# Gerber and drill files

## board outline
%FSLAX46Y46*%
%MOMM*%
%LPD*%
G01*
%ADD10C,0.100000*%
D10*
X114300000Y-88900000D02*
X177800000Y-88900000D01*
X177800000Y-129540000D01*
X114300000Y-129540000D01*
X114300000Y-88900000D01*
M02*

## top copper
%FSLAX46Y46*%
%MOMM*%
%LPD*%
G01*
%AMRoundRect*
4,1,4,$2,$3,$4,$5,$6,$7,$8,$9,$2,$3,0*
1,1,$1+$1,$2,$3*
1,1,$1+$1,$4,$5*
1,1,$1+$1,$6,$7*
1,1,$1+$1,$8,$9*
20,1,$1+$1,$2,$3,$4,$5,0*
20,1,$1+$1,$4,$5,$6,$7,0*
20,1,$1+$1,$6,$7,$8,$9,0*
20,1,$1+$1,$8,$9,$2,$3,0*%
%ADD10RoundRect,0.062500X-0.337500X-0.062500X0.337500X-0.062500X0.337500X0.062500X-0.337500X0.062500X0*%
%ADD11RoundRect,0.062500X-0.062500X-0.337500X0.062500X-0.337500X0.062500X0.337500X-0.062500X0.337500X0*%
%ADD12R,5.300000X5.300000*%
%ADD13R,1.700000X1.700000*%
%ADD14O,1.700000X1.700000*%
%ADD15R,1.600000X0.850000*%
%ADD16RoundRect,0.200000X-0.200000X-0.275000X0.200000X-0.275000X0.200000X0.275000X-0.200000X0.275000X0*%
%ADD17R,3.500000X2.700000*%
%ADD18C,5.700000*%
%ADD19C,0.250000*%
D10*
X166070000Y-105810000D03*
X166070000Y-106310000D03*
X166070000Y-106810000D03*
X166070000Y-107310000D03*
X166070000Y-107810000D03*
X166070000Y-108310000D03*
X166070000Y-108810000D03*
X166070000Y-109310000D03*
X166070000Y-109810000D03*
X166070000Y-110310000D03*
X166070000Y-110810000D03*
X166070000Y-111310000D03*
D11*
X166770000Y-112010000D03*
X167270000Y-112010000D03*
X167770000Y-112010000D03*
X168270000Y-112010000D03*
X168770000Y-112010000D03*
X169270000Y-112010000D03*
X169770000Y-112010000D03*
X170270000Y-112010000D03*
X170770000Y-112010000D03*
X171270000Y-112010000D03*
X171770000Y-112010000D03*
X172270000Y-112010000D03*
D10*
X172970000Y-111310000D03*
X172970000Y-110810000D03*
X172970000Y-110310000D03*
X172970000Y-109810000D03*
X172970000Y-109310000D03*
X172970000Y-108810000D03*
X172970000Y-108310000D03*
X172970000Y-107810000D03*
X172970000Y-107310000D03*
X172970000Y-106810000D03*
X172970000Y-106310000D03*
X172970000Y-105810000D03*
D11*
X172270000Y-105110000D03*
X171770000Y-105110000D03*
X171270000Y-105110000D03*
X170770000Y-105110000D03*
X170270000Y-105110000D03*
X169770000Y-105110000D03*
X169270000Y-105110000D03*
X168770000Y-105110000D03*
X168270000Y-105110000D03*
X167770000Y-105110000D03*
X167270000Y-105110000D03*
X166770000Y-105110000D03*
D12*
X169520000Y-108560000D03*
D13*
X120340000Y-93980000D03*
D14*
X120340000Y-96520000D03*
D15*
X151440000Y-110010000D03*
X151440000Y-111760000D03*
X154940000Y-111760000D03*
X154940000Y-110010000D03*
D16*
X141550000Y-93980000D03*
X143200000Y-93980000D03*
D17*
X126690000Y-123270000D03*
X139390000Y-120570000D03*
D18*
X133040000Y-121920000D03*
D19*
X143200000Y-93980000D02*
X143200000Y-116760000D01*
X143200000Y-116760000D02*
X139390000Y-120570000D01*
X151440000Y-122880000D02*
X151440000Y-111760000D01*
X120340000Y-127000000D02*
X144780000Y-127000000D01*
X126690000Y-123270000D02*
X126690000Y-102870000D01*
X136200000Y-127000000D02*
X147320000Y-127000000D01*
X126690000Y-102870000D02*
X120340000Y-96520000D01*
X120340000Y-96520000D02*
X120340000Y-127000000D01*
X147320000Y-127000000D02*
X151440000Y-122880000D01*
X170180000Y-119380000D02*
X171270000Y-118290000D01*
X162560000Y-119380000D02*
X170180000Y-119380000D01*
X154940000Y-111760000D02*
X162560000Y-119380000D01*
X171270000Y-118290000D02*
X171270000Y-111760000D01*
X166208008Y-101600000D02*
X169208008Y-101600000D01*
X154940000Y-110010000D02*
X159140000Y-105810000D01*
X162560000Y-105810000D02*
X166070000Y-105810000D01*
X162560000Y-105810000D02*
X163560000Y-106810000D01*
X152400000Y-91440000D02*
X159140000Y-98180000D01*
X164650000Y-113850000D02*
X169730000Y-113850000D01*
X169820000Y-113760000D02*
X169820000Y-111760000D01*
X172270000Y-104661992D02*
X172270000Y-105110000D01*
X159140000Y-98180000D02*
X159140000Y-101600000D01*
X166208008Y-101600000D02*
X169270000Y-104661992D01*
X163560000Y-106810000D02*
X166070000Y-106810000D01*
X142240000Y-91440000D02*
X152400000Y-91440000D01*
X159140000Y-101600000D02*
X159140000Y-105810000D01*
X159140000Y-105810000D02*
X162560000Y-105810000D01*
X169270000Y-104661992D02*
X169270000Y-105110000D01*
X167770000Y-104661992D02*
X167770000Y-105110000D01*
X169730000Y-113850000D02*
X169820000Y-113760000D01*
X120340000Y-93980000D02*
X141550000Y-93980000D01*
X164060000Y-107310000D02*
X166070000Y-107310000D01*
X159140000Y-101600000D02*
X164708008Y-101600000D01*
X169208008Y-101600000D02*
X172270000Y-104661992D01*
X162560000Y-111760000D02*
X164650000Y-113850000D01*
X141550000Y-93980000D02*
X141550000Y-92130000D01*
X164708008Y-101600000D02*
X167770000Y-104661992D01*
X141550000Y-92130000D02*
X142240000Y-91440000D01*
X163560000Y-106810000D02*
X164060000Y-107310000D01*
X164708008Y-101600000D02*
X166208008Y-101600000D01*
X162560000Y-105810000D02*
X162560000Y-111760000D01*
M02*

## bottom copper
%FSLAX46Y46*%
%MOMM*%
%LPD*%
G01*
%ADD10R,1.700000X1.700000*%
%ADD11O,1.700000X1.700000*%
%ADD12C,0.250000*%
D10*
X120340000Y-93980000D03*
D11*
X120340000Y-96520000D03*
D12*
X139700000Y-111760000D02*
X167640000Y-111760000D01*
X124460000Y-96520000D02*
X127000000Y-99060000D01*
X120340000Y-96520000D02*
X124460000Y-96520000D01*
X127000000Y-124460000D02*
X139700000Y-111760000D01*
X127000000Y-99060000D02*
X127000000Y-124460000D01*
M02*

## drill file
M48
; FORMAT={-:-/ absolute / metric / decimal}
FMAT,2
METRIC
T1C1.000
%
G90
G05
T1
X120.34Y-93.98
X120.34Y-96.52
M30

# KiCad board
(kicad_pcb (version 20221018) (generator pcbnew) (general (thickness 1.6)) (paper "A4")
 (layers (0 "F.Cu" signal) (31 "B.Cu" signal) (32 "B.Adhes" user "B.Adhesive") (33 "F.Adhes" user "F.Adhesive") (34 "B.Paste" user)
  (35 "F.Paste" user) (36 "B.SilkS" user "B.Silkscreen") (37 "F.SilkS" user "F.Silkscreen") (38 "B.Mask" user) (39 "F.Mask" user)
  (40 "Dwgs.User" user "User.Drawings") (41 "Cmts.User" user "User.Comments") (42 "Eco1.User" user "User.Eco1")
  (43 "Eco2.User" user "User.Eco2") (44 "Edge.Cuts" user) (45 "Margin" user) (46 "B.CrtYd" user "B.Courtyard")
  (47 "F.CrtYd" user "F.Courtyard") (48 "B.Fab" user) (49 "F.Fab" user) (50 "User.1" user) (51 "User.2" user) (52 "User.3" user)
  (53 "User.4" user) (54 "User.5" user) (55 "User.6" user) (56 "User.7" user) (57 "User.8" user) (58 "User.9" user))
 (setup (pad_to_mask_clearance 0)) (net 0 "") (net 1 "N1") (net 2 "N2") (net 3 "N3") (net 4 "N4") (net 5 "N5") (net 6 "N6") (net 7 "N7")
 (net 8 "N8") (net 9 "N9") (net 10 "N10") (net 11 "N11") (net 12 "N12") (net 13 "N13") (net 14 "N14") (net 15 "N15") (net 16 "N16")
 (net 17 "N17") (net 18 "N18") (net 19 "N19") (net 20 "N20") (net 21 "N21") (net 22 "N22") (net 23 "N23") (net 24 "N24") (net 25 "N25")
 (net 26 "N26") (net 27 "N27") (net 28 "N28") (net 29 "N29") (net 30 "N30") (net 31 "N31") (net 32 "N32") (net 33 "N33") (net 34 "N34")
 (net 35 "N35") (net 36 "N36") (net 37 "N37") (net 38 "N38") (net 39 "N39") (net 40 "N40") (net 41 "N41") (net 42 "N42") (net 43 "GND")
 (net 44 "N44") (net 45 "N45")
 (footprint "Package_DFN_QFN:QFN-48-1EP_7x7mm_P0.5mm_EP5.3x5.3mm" (layer "F.Cu") (at 169.52 108.56)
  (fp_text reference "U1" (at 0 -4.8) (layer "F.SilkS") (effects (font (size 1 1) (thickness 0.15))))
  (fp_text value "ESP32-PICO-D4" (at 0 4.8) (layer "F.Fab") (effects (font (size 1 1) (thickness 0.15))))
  (pad "" smd roundrect (at -1.98 -1.98) (size 1.07 1.07) (layers "F.Paste") (roundrect_rratio 0.233645))
  (pad "" smd roundrect (at -1.98 -0.66) (size 1.07 1.07) (layers "F.Paste") (roundrect_rratio 0.233645))
  (pad "" smd roundrect (at -1.98 0.66) (size 1.07 1.07) (layers "F.Paste") (roundrect_rratio 0.233645))
  (pad "" smd roundrect (at -1.98 1.98) (size 1.07 1.07) (layers "F.Paste") (roundrect_rratio 0.233645))
  (pad "" smd roundrect (at -0.66 -1.98) (size 1.07 1.07) (layers "F.Paste") (roundrect_rratio 0.233645))
  (pad "" smd roundrect (at -0.66 -0.66) (size 1.07 1.07) (layers "F.Paste") (roundrect_rratio 0.233645))
  (pad "" smd roundrect (at -0.66 0.66) (size 1.07 1.07) (layers "F.Paste") (roundrect_rratio 0.233645))
  (pad "" smd roundrect (at -0.66 1.98) (size 1.07 1.07) (layers "F.Paste") (roundrect_rratio 0.233645))
  (pad "" smd roundrect (at 0.66 -1.98) (size 1.07 1.07) (layers "F.Paste") (roundrect_rratio 0.233645))
  (pad "" smd roundrect (at 0.66 -0.66) (size 1.07 1.07) (layers "F.Paste") (roundrect_rratio 0.233645))
  (pad "" smd roundrect (at 0.66 0.66) (size 1.07 1.07) (layers "F.Paste") (roundrect_rratio 0.233645))
  (pad "" smd roundrect (at 0.66 1.98) (size 1.07 1.07) (layers "F.Paste") (roundrect_rratio 0.233645))
  (pad "" smd roundrect (at 1.98 -1.98) (size 1.07 1.07) (layers "F.Paste") (roundrect_rratio 0.233645))
  (pad "" smd roundrect (at 1.98 -0.66) (size 1.07 1.07) (layers "F.Paste") (roundrect_rratio 0.233645))
  (pad "" smd roundrect (at 1.98 0.66) (size 1.07 1.07) (layers "F.Paste") (roundrect_rratio 0.233645))
  (pad "" smd roundrect (at 1.98 1.98) (size 1.07 1.07) (layers "F.Paste") (roundrect_rratio 0.233645))
  (pad "1" smd roundrect (at -3.45 -2.75) (size 0.8 0.25) (layers "F.Cu" "F.Paste" "F.Mask") (roundrect_rratio 0.25) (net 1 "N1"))
  (pad "2" smd roundrect (at -3.45 -2.25) (size 0.8 0.25) (layers "F.Cu" "F.Paste" "F.Mask") (roundrect_rratio 0.25) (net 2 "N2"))
  (pad "3" smd roundrect (at -3.45 -1.75) (size 0.8 0.25) (layers "F.Cu" "F.Paste" "F.Mask") (roundrect_rratio 0.25) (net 1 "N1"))
  (pad "4" smd roundrect (at -3.45 -1.25) (size 0.8 0.25) (layers "F.Cu" "F.Paste" "F.Mask") (roundrect_rratio 0.25) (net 1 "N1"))
  (pad "5" smd roundrect (at -3.45 -0.75) (size 0.8 0.25) (layers "F.Cu" "F.Paste" "F.Mask") (roundrect_rratio 0.25) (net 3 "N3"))
  (pad "6" smd roundrect (at -3.45 -0.25) (size 0.8 0.25) (layers "F.Cu" "F.Paste" "F.Mask") (roundrect_rratio 0.25) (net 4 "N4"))
  (pad "7" smd roundrect (at -3.45 0.25) (size 0.8 0.25) (layers "F.Cu" "F.Paste" "F.Mask") (roundrect_rratio 0.25) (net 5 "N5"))
  (pad "8" smd roundrect (at -3.45 0.75) (size 0.8 0.25) (layers "F.Cu" "F.Paste" "F.Mask") (roundrect_rratio 0.25) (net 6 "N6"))
  (pad "9" smd roundrect (at -3.45 1.25) (size 0.8 0.25) (layers "F.Cu" "F.Paste" "F.Mask") (roundrect_rratio 0.25) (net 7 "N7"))
  (pad "10" smd roundrect (at -3.45 1.75) (size 0.8 0.25) (layers "F.Cu" "F.Paste" "F.Mask") (roundrect_rratio 0.25) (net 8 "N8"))
  (pad "11" smd roundrect (at -3.45 2.25) (size 0.8 0.25) (layers "F.Cu" "F.Paste" "F.Mask") (roundrect_rratio 0.25) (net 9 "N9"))
  (pad "12" smd roundrect (at -3.45 2.75) (size 0.8 0.25) (layers "F.Cu" "F.Paste" "F.Mask") (roundrect_rratio 0.25) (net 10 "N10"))
  (pad "13" smd roundrect (at -2.75 3.45) (size 0.25 0.8) (layers "F.Cu" "F.Paste" "F.Mask") (roundrect_rratio 0.25) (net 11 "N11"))
  (pad "14" smd roundrect (at -2.25 3.45) (size 0.25 0.8) (layers "F.Cu" "F.Paste" "F.Mask") (roundrect_rratio 0.25) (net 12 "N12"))
  (pad "15" smd roundrect (at -1.75 3.45) (size 0.25 0.8) (layers "F.Cu" "F.Paste" "F.Mask") (roundrect_rratio 0.25) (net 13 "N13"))
  (pad "16" smd roundrect (at -1.25 3.45) (size 0.25 0.8) (layers "F.Cu" "F.Paste" "F.Mask") (roundrect_rratio 0.25) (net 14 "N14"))
  (pad "17" smd roundrect (at -0.75 3.45) (size 0.25 0.8) (layers "F.Cu" "F.Paste" "F.Mask") (roundrect_rratio 0.25) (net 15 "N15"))
  (pad "18" smd roundrect (at -0.25 3.45) (size 0.25 0.8) (layers "F.Cu" "F.Paste" "F.Mask") (roundrect_rratio 0.25) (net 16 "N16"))
  (pad "19" smd roundrect (at 0.25 3.45) (size 0.25 0.8) (layers "F.Cu" "F.Paste" "F.Mask") (roundrect_rratio 0.25) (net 1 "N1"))
  (pad "20" smd roundrect (at 0.75 3.45) (size 0.25 0.8) (layers "F.Cu" "F.Paste" "F.Mask") (roundrect_rratio 0.25) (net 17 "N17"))
  (pad "21" smd roundrect (at 1.25 3.45) (size 0.25 0.8) (layers "F.Cu" "F.Paste" "F.Mask") (roundrect_rratio 0.25) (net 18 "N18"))
  (pad "22" smd roundrect (at 1.75 3.45) (size 0.25 0.8) (layers "F.Cu" "F.Paste" "F.Mask") (roundrect_rratio 0.25) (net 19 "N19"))
  (pad "23" smd roundrect (at 2.25 3.45) (size 0.25 0.8) (layers "F.Cu" "F.Paste" "F.Mask") (roundrect_rratio 0.25) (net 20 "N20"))
  (pad "24" smd roundrect (at 2.75 3.45) (size 0.25 0.8) (layers "F.Cu" "F.Paste" "F.Mask") (roundrect_rratio 0.25) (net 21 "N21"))
  (pad "25" smd roundrect (at 3.45 2.75) (size 0.8 0.25) (layers "F.Cu" "F.Paste" "F.Mask") (roundrect_rratio 0.25) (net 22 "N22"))
  (pad "26" smd roundrect (at 3.45 2.25) (size 0.8 0.25) (layers "F.Cu" "F.Paste" "F.Mask") (roundrect_rratio 0.25) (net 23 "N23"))
  (pad "27" smd roundrect (at 3.45 1.75) (size 0.8 0.25) (layers "F.Cu" "F.Paste" "F.Mask") (roundrect_rratio 0.25) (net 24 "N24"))
  (pad "28" smd roundrect (at 3.45 1.25) (size 0.8 0.25) (layers "F.Cu" "F.Paste" "F.Mask") (roundrect_rratio 0.25) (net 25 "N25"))
  (pad "29" smd roundrect (at 3.45 0.75) (size 0.8 0.25) (layers "F.Cu" "F.Paste" "F.Mask") (roundrect_rratio 0.25) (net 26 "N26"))
  (pad "30" smd roundrect (at 3.45 0.25) (size 0.8 0.25) (layers "F.Cu" "F.Paste" "F.Mask") (roundrect_rratio 0.25) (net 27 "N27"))
  (pad "31" smd roundrect (at 3.45 -0.25) (size 0.8 0.25) (layers "F.Cu" "F.Paste" "F.Mask") (roundrect_rratio 0.25) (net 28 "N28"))
  (pad "32" smd roundrect (at 3.45 -0.75) (size 0.8 0.25) (layers "F.Cu" "F.Paste" "F.Mask") (roundrect_rratio 0.25) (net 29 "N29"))
  (pad "33" smd roundrect (at 3.45 -1.25) (size 0.8 0.25) (layers "F.Cu" "F.Paste" "F.Mask") (roundrect_rratio 0.25) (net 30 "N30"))
  (pad "34" smd roundrect (at 3.45 -1.75) (size 0.8 0.25) (layers "F.Cu" "F.Paste" "F.Mask") (roundrect_rratio 0.25) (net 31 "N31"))
  (pad "35" smd roundrect (at 3.45 -2.25) (size 0.8 0.25) (layers "F.Cu" "F.Paste" "F.Mask") (roundrect_rratio 0.25) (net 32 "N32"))
  (pad "36" smd roundrect (at 3.45 -2.75) (size 0.8 0.25) (layers "F.Cu" "F.Paste" "F.Mask") (roundrect_rratio 0.25) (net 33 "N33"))
  (pad "37" smd roundrect (at 2.75 -3.45) (size 0.25 0.8) (layers "F.Cu" "F.Paste" "F.Mask") (roundrect_rratio 0.25) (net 1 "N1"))
  (pad "38" smd roundrect (at 2.25 -3.45) (size 0.25 0.8) (layers "F.Cu" "F.Paste" "F.Mask") (roundrect_rratio 0.25) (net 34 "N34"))
  (pad "39" smd roundrect (at 1.75 -3.45) (size 0.25 0.8) (layers "F.Cu" "F.Paste" "F.Mask") (roundrect_rratio 0.25) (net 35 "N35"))
  (pad "40" smd roundrect (at 1.25 -3.45) (size 0.25 0.8) (layers "F.Cu" "F.Paste" "F.Mask") (roundrect_rratio 0.25) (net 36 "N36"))
  (pad "41" smd roundrect (at 0.75 -3.45) (size 0.25 0.8) (layers "F.Cu" "F.Paste" "F.Mask") (roundrect_rratio 0.25) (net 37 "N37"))
  (pad "42" smd roundrect (at 0.25 -3.45) (size 0.25 0.8) (layers "F.Cu" "F.Paste" "F.Mask") (roundrect_rratio 0.25) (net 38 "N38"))
  (pad "43" smd roundrect (at -0.25 -3.45) (size 0.25 0.8) (layers "F.Cu" "F.Paste" "F.Mask") (roundrect_rratio 0.25) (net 1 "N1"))
  (pad "44" smd roundrect (at -0.75 -3.45) (size 0.25 0.8) (layers "F.Cu" "F.Paste" "F.Mask") (roundrect_rratio 0.25) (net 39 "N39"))
  (pad "45" smd roundrect (at -1.25 -3.45) (size 0.25 0.8) (layers "F.Cu" "F.Paste" "F.Mask") (roundrect_rratio 0.25) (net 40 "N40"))
  (pad "46" smd roundrect (at -1.75 -3.45) (size 0.25 0.8) (layers "F.Cu" "F.Paste" "F.Mask") (roundrect_rratio 0.25) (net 1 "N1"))
  (pad "47" smd roundrect (at -2.25 -3.45) (size 0.25 0.8) (layers "F.Cu" "F.Paste" "F.Mask") (roundrect_rratio 0.25) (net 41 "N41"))
  (pad "48" smd roundrect (at -2.75 -3.45) (size 0.25 0.8) (layers "F.Cu" "F.Paste" "F.Mask") (roundrect_rratio 0.25) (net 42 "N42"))
  (pad "49" smd rect (at 0 0) (size 5.3 5.3) (layers "F.Cu" "F.Mask") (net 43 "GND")))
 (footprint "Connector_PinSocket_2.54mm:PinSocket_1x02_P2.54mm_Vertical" (layer "F.Cu") (at 120.34 93.98)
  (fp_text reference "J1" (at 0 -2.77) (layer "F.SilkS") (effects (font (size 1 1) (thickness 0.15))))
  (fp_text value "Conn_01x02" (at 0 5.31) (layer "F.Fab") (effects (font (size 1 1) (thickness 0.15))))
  (pad "1" thru_hole rect (at 0 0) (size 1.7 1.7) (drill 1) (layers "*.Cu" "*.Mask") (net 1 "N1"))
  (pad "2" thru_hole oval (at 0 2.54) (size 1.7 1.7) (drill 1) (layers "*.Cu" "*.Mask") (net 43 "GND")))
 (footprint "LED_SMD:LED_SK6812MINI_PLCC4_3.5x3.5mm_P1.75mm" (layer "F.Cu") (at 153.19 110.885)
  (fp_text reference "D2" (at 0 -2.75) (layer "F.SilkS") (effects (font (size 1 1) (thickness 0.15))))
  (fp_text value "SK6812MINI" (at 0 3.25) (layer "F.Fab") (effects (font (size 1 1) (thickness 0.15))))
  (pad "1" smd rect (at -1.75 -0.875) (size 1.6 0.85) (layers "F.Cu" "F.Paste" "F.Mask") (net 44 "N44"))
  (pad "2" smd rect (at -1.75 0.875) (size 1.6 0.85) (layers "F.Cu" "F.Paste" "F.Mask") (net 43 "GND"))
  (pad "3" smd rect (at 1.75 0.875) (size 1.6 0.85) (layers "F.Cu" "F.Paste" "F.Mask") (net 19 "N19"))
  (pad "4" smd rect (at 1.75 -0.875) (size 1.6 0.85) (layers "F.Cu" "F.Paste" "F.Mask") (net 1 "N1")))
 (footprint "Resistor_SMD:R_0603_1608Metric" (layer "F.Cu") (at 142.375 93.98)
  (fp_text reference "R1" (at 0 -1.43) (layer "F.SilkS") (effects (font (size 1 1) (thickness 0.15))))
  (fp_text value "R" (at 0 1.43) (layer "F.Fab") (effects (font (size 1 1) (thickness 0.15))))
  (pad "1" smd roundrect (at -0.825 0) (size 0.8 0.95) (layers "F.Cu" "F.Paste" "F.Mask") (roundrect_rratio 0.25) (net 1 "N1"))
  (pad "2" smd roundrect (at 0.825 0) (size 0.8 0.95) (layers "F.Cu" "F.Paste" "F.Mask") (roundrect_rratio 0.25) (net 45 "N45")))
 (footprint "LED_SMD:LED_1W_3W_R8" (layer "F.Cu") (at 133.04 121.92)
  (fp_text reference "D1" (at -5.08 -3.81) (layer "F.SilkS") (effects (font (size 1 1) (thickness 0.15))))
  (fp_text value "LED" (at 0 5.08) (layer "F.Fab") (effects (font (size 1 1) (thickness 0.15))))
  (pad "1" smd rect (at -6.35 1.35) (size 3.5 2.7) (layers "F.Cu" "F.Paste" "F.Mask") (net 43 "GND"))
  (pad "2" smd rect (at 6.35 -1.35) (size 3.5 2.7) (layers "F.Cu" "F.Paste" "F.Mask") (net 45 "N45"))
  (pad "3" smd circle (at 0 0) (size 5.7 5.7) (layers "F.Cu" "F.Paste" "F.Mask")))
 (gr_rect (start 114.3 88.9) (end 177.8 129.54) (stroke (width 0.1) (type default)) (fill none) (layer "Edge.Cuts"))
 (segment (start 143.2 93.98) (end 143.2 116.76) (width 0.25) (layer "F.Cu") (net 45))
 (segment (start 143.2 116.76) (end 139.39 120.57) (width 0.25) (layer "F.Cu") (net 45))
 (segment (start 151.44 122.88) (end 151.44 111.76) (width 0.25) (layer "F.Cu") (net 43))
 (segment (start 120.34 127) (end 144.78 127) (width 0.25) (layer "F.Cu") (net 43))
 (segment (start 126.69 123.27) (end 126.69 102.87) (width 0.25) (layer "F.Cu") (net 43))
 (segment (start 136.2 127) (end 147.32 127) (width 0.25) (layer "F.Cu") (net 43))
 (segment (start 126.69 102.87) (end 120.34 96.52) (width 0.25) (layer "F.Cu") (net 43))
 (segment (start 120.34 96.52) (end 120.34 127) (width 0.25) (layer "F.Cu") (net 43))
 (segment (start 147.32 127) (end 151.44 122.88) (width 0.25) (layer "F.Cu") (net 43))
 (segment (start 139.7 111.76) (end 167.64 111.76) (width 0.25) (layer "B.Cu") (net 43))
 (segment (start 124.46 96.52) (end 127 99.06) (width 0.25) (layer "B.Cu") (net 43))
 (segment (start 120.34 96.52) (end 124.46 96.52) (width 0.25) (layer "B.Cu") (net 43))
 (segment (start 127 124.46) (end 139.7 111.76) (width 0.25) (layer "B.Cu") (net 43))
 (segment (start 127 99.06) (end 127 124.46) (width 0.25) (layer "B.Cu") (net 43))
 (segment (start 170.18 119.38) (end 171.27 118.29) (width 0.25) (layer "F.Cu") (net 19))
 (segment (start 162.56 119.38) (end 170.18 119.38) (width 0.25) (layer "F.Cu") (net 19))
 (segment (start 154.94 111.76) (end 162.56 119.38) (width 0.25) (layer "F.Cu") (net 19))
 (segment (start 171.27 118.29) (end 171.27 111.76) (width 0.25) (layer "F.Cu") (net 19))
 (segment (start 166.208008 101.6) (end 169.208008 101.6) (width 0.25) (layer "F.Cu") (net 1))
 (segment (start 154.94 110.01) (end 159.14 105.81) (width 0.25) (layer "F.Cu") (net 1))
 (segment (start 162.56 105.81) (end 166.07 105.81) (width 0.25) (layer "F.Cu") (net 1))
 (segment (start 162.56 105.81) (end 163.56 106.81) (width 0.25) (layer "F.Cu") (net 1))
 (segment (start 152.4 91.44) (end 159.14 98.18) (width 0.25) (layer "F.Cu") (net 1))
 (segment (start 164.65 113.85) (end 169.73 113.85) (width 0.25) (layer "F.Cu") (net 1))
 (segment (start 169.82 113.76) (end 169.82 111.76) (width 0.25) (layer "F.Cu") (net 1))
 (segment (start 172.27 104.661992) (end 172.27 105.11) (width 0.25) (layer "F.Cu") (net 1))
 (segment (start 159.14 98.18) (end 159.14 101.6) (width 0.25) (layer "F.Cu") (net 1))
 (segment (start 166.208008 101.6) (end 169.27 104.661992) (width 0.25) (layer "F.Cu") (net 1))
 (segment (start 163.56 106.81) (end 166.07 106.81) (width 0.25) (layer "F.Cu") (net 1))
 (segment (start 142.24 91.44) (end 152.4 91.44) (width 0.25) (layer "F.Cu") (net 1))
 (segment (start 159.14 101.6) (end 159.14 105.81) (width 0.25) (layer "F.Cu") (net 1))
 (segment (start 159.14 105.81) (end 162.56 105.81) (width 0.25) (layer "F.Cu") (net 1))
 (segment (start 169.27 104.661992) (end 169.27 105.11) (width 0.25) (layer "F.Cu") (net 1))
 (segment (start 167.77 104.661992) (end 167.77 105.11) (width 0.25) (layer "F.Cu") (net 1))
 (segment (start 169.73 113.85) (end 169.82 113.76) (width 0.25) (layer "F.Cu") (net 1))
 (segment (start 120.34 93.98) (end 141.55 93.98) (width 0.25) (layer "F.Cu") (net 1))
 (segment (start 164.06 107.31) (end 166.07 107.31) (width 0.25) (layer "F.Cu") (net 1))
 (segment (start 159.14 101.6) (end 164.708008 101.6) (width 0.25) (layer "F.Cu") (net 1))
 (segment (start 169.208008 101.6) (end 172.27 104.661992) (width 0.25) (layer "F.Cu") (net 1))
 (segment (start 162.56 111.76) (end 164.65 113.85) (width 0.25) (layer "F.Cu") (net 1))
 (segment (start 141.55 93.98) (end 141.55 92.13) (width 0.25) (layer "F.Cu") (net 1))
 (segment (start 164.708008 101.6) (end 167.77 104.661992) (width 0.25) (layer "F.Cu") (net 1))
 (segment (start 141.55 92.13) (end 142.24 91.44) (width 0.25) (layer "F.Cu") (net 1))
 (segment (start 163.56 106.81) (end 164.06 107.31) (width 0.25) (layer "F.Cu") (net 1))
 (segment (start 164.708008 101.6) (end 166.208008 101.6) (width 0.25) (layer "F.Cu") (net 1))
 (segment (start 162.56 105.81) (end 162.56 111.76) (width 0.25) (layer "F.Cu") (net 1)))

